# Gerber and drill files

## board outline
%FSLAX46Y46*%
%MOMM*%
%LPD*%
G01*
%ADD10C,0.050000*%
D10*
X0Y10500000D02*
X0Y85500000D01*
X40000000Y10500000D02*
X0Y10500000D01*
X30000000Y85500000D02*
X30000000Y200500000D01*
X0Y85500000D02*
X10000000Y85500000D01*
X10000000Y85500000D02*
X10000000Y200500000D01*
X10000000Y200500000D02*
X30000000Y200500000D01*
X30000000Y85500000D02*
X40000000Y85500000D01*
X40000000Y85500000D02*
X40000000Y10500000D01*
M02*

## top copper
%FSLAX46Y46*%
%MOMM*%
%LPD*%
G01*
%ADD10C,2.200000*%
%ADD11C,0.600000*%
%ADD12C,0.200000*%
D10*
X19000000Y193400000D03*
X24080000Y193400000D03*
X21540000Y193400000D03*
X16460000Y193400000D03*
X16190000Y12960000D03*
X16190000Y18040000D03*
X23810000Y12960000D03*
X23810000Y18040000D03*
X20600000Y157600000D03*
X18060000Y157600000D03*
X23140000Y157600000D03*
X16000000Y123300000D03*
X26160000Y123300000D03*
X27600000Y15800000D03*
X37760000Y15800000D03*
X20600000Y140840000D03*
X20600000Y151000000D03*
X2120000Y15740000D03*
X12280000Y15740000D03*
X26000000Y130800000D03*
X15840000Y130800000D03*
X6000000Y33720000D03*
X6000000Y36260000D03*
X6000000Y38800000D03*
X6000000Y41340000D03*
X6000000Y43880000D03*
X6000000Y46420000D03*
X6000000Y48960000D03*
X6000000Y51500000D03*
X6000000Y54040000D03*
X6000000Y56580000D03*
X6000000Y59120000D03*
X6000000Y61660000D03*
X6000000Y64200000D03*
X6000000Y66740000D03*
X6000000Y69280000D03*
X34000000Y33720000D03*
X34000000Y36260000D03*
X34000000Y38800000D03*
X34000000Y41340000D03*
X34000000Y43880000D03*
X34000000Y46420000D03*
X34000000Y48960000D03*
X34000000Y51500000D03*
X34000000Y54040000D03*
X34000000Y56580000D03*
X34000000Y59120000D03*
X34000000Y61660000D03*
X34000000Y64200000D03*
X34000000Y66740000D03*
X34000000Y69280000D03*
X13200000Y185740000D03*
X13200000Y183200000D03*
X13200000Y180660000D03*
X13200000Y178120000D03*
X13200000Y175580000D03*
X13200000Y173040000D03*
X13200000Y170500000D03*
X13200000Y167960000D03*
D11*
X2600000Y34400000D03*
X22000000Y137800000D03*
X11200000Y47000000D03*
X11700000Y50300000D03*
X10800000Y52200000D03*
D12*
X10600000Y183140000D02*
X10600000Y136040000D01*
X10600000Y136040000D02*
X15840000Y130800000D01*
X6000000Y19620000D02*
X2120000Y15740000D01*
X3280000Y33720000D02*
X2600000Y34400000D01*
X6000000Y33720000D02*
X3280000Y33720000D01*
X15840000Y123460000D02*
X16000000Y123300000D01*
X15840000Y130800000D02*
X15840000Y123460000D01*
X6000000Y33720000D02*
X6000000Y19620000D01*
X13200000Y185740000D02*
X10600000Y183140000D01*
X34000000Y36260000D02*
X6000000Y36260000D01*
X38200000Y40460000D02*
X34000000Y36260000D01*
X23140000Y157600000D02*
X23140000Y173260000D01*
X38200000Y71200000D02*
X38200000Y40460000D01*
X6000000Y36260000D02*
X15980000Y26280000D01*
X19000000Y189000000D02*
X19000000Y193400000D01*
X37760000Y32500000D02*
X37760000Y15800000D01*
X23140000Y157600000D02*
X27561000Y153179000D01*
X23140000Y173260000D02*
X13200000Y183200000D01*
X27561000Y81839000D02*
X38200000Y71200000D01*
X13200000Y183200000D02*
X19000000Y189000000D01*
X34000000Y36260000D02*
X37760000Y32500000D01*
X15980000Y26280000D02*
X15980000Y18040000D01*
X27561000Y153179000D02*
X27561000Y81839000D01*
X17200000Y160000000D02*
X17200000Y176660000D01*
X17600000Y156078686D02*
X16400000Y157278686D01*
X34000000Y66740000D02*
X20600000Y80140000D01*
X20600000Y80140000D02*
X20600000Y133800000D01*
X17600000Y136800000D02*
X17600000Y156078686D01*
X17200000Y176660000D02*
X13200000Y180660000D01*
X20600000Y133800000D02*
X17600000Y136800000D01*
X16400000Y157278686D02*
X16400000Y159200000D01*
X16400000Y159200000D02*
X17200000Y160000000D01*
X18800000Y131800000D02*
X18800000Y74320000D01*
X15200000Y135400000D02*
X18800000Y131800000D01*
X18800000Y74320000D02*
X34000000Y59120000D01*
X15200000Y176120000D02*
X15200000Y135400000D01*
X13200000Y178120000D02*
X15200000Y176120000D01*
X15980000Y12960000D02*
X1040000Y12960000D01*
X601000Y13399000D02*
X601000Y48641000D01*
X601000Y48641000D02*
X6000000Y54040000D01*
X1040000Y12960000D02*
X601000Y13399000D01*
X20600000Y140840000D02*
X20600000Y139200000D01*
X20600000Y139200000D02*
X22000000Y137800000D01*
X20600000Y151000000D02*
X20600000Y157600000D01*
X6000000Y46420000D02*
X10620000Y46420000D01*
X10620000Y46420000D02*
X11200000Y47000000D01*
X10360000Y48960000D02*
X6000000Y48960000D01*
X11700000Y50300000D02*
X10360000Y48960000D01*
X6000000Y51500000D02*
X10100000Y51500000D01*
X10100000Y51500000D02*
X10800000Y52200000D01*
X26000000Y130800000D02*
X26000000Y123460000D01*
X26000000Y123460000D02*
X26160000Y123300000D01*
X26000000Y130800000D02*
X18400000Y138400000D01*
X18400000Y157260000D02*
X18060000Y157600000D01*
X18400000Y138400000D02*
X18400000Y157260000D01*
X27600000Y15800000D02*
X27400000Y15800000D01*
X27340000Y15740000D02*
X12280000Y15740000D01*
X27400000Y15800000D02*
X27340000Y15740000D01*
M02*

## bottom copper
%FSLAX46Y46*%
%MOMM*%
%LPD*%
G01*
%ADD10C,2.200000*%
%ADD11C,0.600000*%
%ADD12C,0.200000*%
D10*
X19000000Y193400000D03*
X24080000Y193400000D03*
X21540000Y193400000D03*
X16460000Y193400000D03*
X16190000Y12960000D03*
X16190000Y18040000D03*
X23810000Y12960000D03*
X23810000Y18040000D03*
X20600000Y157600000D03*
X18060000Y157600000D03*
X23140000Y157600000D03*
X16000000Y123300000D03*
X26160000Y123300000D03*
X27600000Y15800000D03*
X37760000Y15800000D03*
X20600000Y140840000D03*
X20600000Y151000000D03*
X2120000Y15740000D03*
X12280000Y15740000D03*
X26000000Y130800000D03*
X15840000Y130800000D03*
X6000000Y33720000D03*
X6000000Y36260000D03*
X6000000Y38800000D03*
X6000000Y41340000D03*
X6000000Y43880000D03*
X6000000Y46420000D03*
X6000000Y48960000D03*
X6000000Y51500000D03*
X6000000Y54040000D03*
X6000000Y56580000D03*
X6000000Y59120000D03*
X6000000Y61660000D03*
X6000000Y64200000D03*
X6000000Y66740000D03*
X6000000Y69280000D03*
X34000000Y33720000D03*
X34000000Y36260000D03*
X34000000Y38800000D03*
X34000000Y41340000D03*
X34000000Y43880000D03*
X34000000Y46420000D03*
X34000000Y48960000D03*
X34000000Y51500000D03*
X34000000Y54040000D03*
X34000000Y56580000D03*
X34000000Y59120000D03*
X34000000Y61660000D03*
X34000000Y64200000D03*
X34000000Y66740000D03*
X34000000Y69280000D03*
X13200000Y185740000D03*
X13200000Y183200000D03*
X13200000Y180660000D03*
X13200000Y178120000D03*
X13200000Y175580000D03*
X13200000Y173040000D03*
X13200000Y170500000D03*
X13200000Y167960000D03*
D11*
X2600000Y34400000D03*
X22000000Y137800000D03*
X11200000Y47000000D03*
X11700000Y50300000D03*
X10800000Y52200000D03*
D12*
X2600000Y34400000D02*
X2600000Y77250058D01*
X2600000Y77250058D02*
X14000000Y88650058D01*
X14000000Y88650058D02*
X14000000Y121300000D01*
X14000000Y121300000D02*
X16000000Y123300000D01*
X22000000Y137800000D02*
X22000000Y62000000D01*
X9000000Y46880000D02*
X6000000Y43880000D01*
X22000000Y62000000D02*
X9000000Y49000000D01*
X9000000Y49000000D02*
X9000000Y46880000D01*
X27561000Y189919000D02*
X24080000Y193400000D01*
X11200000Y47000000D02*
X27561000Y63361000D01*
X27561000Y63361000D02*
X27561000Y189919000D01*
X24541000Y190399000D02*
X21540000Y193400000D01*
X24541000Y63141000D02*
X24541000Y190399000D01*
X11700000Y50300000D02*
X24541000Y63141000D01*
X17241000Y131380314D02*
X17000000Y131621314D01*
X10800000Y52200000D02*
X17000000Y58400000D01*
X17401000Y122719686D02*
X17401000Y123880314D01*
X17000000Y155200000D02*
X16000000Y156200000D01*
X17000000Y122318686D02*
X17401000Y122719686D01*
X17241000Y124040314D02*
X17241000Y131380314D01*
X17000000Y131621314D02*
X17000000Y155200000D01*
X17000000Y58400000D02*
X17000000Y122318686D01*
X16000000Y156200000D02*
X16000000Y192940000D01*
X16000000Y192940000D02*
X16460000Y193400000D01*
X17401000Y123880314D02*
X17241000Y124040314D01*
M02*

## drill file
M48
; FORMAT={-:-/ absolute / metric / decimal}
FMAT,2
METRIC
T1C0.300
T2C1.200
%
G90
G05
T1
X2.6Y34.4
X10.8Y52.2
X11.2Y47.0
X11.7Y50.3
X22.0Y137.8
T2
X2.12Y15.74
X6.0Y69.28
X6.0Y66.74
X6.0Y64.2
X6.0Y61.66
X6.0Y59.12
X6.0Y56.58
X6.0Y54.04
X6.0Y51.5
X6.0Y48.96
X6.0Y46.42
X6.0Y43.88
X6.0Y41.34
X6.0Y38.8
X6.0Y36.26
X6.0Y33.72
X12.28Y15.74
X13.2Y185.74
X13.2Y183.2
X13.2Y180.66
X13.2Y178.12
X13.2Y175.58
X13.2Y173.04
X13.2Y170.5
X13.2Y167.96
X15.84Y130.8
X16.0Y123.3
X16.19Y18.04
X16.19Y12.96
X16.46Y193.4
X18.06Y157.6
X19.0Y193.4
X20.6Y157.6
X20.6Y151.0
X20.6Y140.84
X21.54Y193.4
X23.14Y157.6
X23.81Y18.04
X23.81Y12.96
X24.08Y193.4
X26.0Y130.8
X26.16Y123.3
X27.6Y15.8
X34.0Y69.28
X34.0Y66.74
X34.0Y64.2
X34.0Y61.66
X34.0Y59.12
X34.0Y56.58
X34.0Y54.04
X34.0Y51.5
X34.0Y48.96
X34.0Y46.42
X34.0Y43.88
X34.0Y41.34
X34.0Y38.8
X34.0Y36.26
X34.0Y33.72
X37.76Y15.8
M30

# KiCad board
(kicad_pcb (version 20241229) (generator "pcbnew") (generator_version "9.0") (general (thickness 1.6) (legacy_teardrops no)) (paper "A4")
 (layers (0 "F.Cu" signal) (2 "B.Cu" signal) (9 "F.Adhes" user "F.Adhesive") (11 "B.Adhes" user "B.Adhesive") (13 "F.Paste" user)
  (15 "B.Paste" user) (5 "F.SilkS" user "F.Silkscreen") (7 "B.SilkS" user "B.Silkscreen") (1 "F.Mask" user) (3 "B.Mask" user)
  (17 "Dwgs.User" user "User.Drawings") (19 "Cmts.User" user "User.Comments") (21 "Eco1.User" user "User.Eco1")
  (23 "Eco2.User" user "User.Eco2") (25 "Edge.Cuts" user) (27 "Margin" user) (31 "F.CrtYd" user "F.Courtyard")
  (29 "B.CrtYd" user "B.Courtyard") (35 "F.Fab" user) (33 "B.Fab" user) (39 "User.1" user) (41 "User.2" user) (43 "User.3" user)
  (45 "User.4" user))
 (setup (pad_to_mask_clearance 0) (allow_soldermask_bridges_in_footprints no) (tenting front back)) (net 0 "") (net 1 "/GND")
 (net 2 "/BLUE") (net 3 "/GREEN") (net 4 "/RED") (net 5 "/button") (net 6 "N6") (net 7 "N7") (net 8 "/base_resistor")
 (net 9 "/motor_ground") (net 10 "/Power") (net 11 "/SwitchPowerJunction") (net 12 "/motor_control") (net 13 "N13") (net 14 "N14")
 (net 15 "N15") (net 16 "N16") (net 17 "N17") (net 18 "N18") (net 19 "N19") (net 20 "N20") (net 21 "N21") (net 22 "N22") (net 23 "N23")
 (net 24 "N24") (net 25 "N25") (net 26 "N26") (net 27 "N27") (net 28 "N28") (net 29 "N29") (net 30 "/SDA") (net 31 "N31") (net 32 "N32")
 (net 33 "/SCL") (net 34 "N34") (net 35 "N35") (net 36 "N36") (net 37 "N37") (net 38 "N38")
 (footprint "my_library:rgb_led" (layer "F.Cu") (at 16.46 -193.4)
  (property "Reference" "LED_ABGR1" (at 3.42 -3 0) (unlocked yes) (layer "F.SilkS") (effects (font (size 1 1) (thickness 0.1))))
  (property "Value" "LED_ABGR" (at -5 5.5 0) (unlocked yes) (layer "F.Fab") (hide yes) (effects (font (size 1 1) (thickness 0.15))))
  (pad "1" thru_hole circle (at 2.54 0) (size 2.2 2.2) (drill 1.2) (layers "*.Cu" "*.Mask") (remove_unused_layers no) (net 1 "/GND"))
  (pad "2" thru_hole circle (at 7.62 0) (size 2.2 2.2) (drill 1.2) (layers "*.Cu" "*.Mask") (remove_unused_layers no) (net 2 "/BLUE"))
  (pad "3" thru_hole circle (at 5.08 0) (size 2.2 2.2) (drill 1.2) (layers "*.Cu" "*.Mask") (remove_unused_layers no) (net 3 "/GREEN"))
  (pad "4" thru_hole circle (at 0 0) (size 2.2 2.2) (drill 1.2) (layers "*.Cu" "*.Mask") (remove_unused_layers no) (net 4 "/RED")))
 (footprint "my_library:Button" (layer "F.Cu") (at 16.19 -12.96 90)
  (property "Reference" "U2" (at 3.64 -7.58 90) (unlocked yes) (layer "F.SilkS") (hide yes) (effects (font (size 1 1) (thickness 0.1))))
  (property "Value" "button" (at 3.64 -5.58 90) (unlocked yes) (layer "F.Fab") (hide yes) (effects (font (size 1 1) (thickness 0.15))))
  (pad "1" thru_hole circle (at 0 0 90) (size 2.2 2.2) (drill 1.2) (layers "*.Cu" "*.Mask") (remove_unused_layers no) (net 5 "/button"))
  (pad "2" thru_hole circle (at 5.08 0 90) (size 2.2 2.2) (drill 1.2) (layers "*.Cu" "*.Mask") (remove_unused_layers no) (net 1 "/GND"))
  (pad "3" thru_hole circle (at 0 7.62 90) (size 2.2 2.2) (drill 1.2) (layers "*.Cu" "*.Mask") (remove_unused_layers no) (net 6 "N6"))
  (pad "4" thru_hole circle (at 5.08 7.62 90) (size 2.2 2.2) (drill 1.2) (layers "*.Cu" "*.Mask") (remove_unused_layers no) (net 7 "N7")))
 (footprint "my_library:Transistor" (layer "F.Cu") (at 18.06 -157.6 90)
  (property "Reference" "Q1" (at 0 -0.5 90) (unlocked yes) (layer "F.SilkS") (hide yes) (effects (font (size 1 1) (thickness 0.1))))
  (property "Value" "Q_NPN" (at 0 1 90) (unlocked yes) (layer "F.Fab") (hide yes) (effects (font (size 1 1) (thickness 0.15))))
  (pad "B" thru_hole circle (at 0 2.54 90) (size 2.2 2.2) (drill 1.2) (layers "*.Cu" "*.Mask") (remove_unused_layers no)
   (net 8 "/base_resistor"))
  (pad "C" thru_hole circle (at 0 0 90) (size 2.2 2.2) (drill 1.2) (layers "*.Cu" "*.Mask") (remove_unused_layers no)
   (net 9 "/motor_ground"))
  (pad "E" thru_hole circle (at 0 5.08 90) (size 2.2 2.2) (drill 1.2) (layers "*.Cu" "*.Mask") (remove_unused_layers no) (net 1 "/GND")))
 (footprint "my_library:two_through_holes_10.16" (layer "F.Cu") (at 16 -123.3)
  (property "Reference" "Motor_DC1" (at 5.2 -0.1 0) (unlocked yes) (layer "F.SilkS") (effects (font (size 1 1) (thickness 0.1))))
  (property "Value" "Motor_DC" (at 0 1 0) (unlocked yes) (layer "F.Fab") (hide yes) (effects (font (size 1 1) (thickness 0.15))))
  (pad "1" thru_hole circle (at 0 0) (size 2.2 2.2) (drill 1.2) (layers "*.Cu" "*.Mask") (remove_unused_layers no) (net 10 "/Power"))
  (pad "2" thru_hole circle (at 10.16 0) (size 2.2 2.2) (drill 1.2) (layers "*.Cu" "*.Mask") (remove_unused_layers no)
   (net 9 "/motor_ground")))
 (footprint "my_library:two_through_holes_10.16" (layer "F.Cu") (at 27.6 -15.8)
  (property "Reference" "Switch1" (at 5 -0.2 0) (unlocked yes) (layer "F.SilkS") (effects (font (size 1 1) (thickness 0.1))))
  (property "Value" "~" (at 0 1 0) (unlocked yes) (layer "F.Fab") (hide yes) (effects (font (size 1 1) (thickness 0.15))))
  (pad "1" thru_hole circle (at 0 0) (size 2.2 2.2) (drill 1.2) (layers "*.Cu" "*.Mask") (remove_unused_layers no)
   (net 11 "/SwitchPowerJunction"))
  (pad "2" thru_hole circle (at 10.16 0) (size 2.2 2.2) (drill 1.2) (layers "*.Cu" "*.Mask") (remove_unused_layers no) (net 1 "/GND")))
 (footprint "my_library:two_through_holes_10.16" (layer "F.Cu") (at 20.6 -140.84 90)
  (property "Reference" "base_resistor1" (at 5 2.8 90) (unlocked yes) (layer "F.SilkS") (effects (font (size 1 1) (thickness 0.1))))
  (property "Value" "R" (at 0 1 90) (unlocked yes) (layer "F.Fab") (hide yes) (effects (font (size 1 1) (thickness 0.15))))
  (pad "1" thru_hole circle (at 0 0 90) (size 2.2 2.2) (drill 1.2) (layers "*.Cu" "*.Mask") (remove_unused_layers no)
   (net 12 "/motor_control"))
  (pad "2" thru_hole circle (at 10.16 0 90) (size 2.2 2.2) (drill 1.2) (layers "*.Cu" "*.Mask") (remove_unused_layers no)
   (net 8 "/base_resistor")))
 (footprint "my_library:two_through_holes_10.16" (layer "F.Cu") (at 2.12 -15.74)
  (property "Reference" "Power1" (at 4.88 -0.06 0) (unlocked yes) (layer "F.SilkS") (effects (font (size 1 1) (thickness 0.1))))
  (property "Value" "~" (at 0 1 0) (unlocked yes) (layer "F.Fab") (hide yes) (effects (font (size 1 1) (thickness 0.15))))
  (pad "1" thru_hole circle (at 0 0) (size 2.2 2.2) (drill 1.2) (layers "*.Cu" "*.Mask") (remove_unused_layers no) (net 10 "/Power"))
  (pad "2" thru_hole circle (at 10.16 0) (size 2.2 2.2) (drill 1.2) (layers "*.Cu" "*.Mask") (remove_unused_layers no)
   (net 11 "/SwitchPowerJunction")))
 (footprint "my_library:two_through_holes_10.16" (layer "F.Cu") (at 26 -130.8 180)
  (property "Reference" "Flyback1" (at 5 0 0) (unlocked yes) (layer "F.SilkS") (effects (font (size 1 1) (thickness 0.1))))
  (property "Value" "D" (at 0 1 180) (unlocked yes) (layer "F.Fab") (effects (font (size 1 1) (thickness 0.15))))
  (pad "1" thru_hole circle (at 0 0 180) (size 2.2 2.2) (drill 1.2) (layers "*.Cu" "*.Mask") (remove_unused_layers no)
   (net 9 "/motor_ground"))
  (pad "2" thru_hole circle (at 10.16 0 180) (size 2.2 2.2) (drill 1.2) (layers "*.Cu" "*.Mask") (remove_unused_layers no) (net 10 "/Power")))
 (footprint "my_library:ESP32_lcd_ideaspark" (layer "F.Cu") (at 20 -51.5)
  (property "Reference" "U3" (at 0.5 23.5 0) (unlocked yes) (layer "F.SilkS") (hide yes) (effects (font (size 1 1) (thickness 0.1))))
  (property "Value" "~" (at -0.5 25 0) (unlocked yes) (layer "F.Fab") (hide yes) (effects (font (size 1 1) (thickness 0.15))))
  (pad "1" thru_hole circle (at -14 17.78) (size 2.2 2.2) (drill 1.2) (layers "*.Cu" "*.Mask") (remove_unused_layers no) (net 10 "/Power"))
  (pad "2" thru_hole circle (at -14 15.24) (size 2.2 2.2) (drill 1.2) (layers "*.Cu" "*.Mask") (remove_unused_layers no) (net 1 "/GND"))
  (pad "3" thru_hole circle (at -14 12.7) (size 2.2 2.2) (drill 1.2) (layers "*.Cu" "*.Mask") (remove_unused_layers no) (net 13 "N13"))
  (pad "4" thru_hole circle (at -14 10.16) (size 2.2 2.2) (drill 1.2) (layers "*.Cu" "*.Mask") (remove_unused_layers no) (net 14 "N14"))
  (pad "5" thru_hole circle (at -14 7.62) (size 2.2 2.2) (drill 1.2) (layers "*.Cu" "*.Mask") (remove_unused_layers no)
   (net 12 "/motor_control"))
  (pad "6" thru_hole circle (at -14 5.08) (size 2.2 2.2) (drill 1.2) (layers "*.Cu" "*.Mask") (remove_unused_layers no) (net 2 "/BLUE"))
  (pad "7" thru_hole circle (at -14 2.54) (size 2.2 2.2) (drill 1.2) (layers "*.Cu" "*.Mask") (remove_unused_layers no) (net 3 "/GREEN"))
  (pad "8" thru_hole circle (at -14 0) (size 2.2 2.2) (drill 1.2) (layers "*.Cu" "*.Mask") (remove_unused_layers no) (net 4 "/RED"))
  (pad "9" thru_hole circle (at -14 -2.54) (size 2.2 2.2) (drill 1.2) (layers "*.Cu" "*.Mask") (remove_unused_layers no) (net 5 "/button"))
  (pad "10" thru_hole circle (at -14 -5.08) (size 2.2 2.2) (drill 1.2) (layers "*.Cu" "*.Mask") (remove_unused_layers no) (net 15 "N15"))
  (pad "11" thru_hole circle (at -14 -7.62) (size 2.2 2.2) (drill 1.2) (layers "*.Cu" "*.Mask") (remove_unused_layers no) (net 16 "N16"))
  (pad "12" thru_hole circle (at -14 -10.16) (size 2.2 2.2) (drill 1.2) (layers "*.Cu" "*.Mask") (remove_unused_layers no) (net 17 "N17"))
  (pad "13" thru_hole circle (at -14 -12.7) (size 2.2 2.2) (drill 1.2) (layers "*.Cu" "*.Mask") (remove_unused_layers no) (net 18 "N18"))
  (pad "14" thru_hole circle (at -14 -15.24) (size 2.2 2.2) (drill 1.2) (layers "*.Cu" "*.Mask") (remove_unused_layers no) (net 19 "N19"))
  (pad "15" thru_hole circle (at -14 -17.78) (size 2.2 2.2) (drill 1.2) (layers "*.Cu" "*.Mask") (remove_unused_layers no) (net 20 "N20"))
  (pad "16" thru_hole circle (at 14 17.78) (size 2.2 2.2) (drill 1.2) (layers "*.Cu" "*.Mask") (remove_unused_layers no) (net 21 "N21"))
  (pad "17" thru_hole circle (at 14 15.24) (size 2.2 2.2) (drill 1.2) (layers "*.Cu" "*.Mask") (remove_unused_layers no) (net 1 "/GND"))
  (pad "18" thru_hole circle (at 14 12.7) (size 2.2 2.2) (drill 1.2) (layers "*.Cu" "*.Mask") (remove_unused_layers no) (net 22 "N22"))
  (pad "19" thru_hole circle (at 14 10.16) (size 2.2 2.2) (drill 1.2) (layers "*.Cu" "*.Mask") (remove_unused_layers no) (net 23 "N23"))
  (pad "20" thru_hole circle (at 14 7.62) (size 2.2 2.2) (drill 1.2) (layers "*.Cu" "*.Mask") (remove_unused_layers no) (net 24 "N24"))
  (pad "21" thru_hole circle (at 14 5.08) (size 2.2 2.2) (drill 1.2) (layers "*.Cu" "*.Mask") (remove_unused_layers no) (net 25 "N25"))
  (pad "22" thru_hole circle (at 14 2.54) (size 2.2 2.2) (drill 1.2) (layers "*.Cu" "*.Mask") (remove_unused_layers no) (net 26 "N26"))
  (pad "23" thru_hole circle (at 14 0) (size 2.2 2.2) (drill 1.2) (layers "*.Cu" "*.Mask") (remove_unused_layers no) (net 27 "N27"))
  (pad "24" thru_hole circle (at 14 -2.54) (size 2.2 2.2) (drill 1.2) (layers "*.Cu" "*.Mask") (remove_unused_layers no) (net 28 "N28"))
  (pad "25" thru_hole circle (at 14 -5.08) (size 2.2 2.2) (drill 1.2) (layers "*.Cu" "*.Mask") (remove_unused_layers no) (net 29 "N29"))
  (pad "26" thru_hole circle (at 14 -7.62) (size 2.2 2.2) (drill 1.2) (layers "*.Cu" "*.Mask") (remove_unused_layers no) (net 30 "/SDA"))
  (pad "27" thru_hole circle (at 14 -10.16) (size 2.2 2.2) (drill 1.2) (layers "*.Cu" "*.Mask") (remove_unused_layers no) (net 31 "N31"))
  (pad "28" thru_hole circle (at 14 -12.7) (size 2.2 2.2) (drill 1.2) (layers "*.Cu" "*.Mask") (remove_unused_layers no) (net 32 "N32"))
  (pad "29" thru_hole circle (at 14 -15.24) (size 2.2 2.2) (drill 1.2) (layers "*.Cu" "*.Mask") (remove_unused_layers no) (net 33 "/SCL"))
  (pad "30" thru_hole circle (at 14 -17.78) (size 2.2 2.2) (drill 1.2) (layers "*.Cu" "*.Mask") (remove_unused_layers no) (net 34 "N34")))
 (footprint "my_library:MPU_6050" (layer "F.Cu") (at 13.2 -185.74)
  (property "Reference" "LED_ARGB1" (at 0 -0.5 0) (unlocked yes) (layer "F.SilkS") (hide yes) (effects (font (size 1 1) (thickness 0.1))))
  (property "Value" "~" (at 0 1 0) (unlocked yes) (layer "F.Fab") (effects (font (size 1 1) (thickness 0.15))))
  (pad "1" thru_hole circle (at 0 0) (size 2.2 2.2) (drill 1.2) (layers "*.Cu" "*.Mask") (remove_unused_layers no) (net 10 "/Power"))
  (pad "2" thru_hole circle (at 0 2.54) (size 2.2 2.2) (drill 1.2) (layers "*.Cu" "*.Mask") (remove_unused_layers no) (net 1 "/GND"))
  (pad "3" thru_hole circle (at 0 5.08) (size 2.2 2.2) (drill 1.2) (layers "*.Cu" "*.Mask") (remove_unused_layers no) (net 33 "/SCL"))
  (pad "4" thru_hole circle (at 0 7.62) (size 2.2 2.2) (drill 1.2) (layers "*.Cu" "*.Mask") (remove_unused_layers no) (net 30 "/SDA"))
  (pad "5" thru_hole circle (at 0 10.16) (size 2.2 2.2) (drill 1.2) (layers "*.Cu" "*.Mask") (remove_unused_layers no) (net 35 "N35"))
  (pad "6" thru_hole circle (at 0 12.7) (size 2.2 2.2) (drill 1.2) (layers "*.Cu" "*.Mask") (remove_unused_layers no) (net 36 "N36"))
  (pad "7" thru_hole circle (at 0 15.24) (size 2.2 2.2) (drill 1.2) (layers "*.Cu" "*.Mask") (remove_unused_layers no) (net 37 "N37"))
  (pad "8" thru_hole circle (at 0 17.78) (size 2.2 2.2) (drill 1.2) (layers "*.Cu" "*.Mask") (remove_unused_layers no) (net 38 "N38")))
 (gr_line (start 0 -10.5) (end 0 -85.5) (stroke (width 0.05) (type solid)) (layer "Edge.Cuts"))
 (gr_line (start 40 -10.5) (end 0 -10.5) (stroke (width 0.05) (type solid)) (layer "Edge.Cuts"))
 (gr_line (start 30 -85.5) (end 30 -200.5) (stroke (width 0.05) (type solid)) (layer "Edge.Cuts"))
 (gr_line (start 0 -85.5) (end 10 -85.5) (stroke (width 0.05) (type default)) (layer "Edge.Cuts"))
 (gr_line (start 10 -85.5) (end 10 -200.5) (stroke (width 0.05) (type solid)) (layer "Edge.Cuts"))
 (gr_line (start 10 -200.5) (end 30 -200.5) (stroke (width 0.05) (type solid)) (layer "Edge.Cuts"))
 (gr_line (start 30 -85.5) (end 40 -85.5) (stroke (width 0.05) (type default)) (layer "Edge.Cuts"))
 (gr_line (start 40 -85.5) (end 40 -10.5) (stroke (width 0.05) (type solid)) (layer "Edge.Cuts"))
 (segment (start 10.6 -183.14) (end 10.6 -136.04) (width 0.2) (layer "F.Cu") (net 10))
 (segment (start 10.6 -136.04) (end 15.84 -130.8) (width 0.2) (layer "F.Cu") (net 10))
 (segment (start 6 -19.62) (end 2.12 -15.74) (width 0.2) (layer "F.Cu") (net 10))
 (segment (start 3.28 -33.72) (end 2.6 -34.4) (width 0.2) (layer "F.Cu") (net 10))
 (segment (start 6 -33.72) (end 3.28 -33.72) (width 0.2) (layer "F.Cu") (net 10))
 (segment (start 15.84 -123.46) (end 16 -123.3) (width 0.2) (layer "F.Cu") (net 10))
 (segment (start 15.84 -130.8) (end 15.84 -123.46) (width 0.2) (layer "F.Cu") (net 10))
 (segment (start 6 -33.72) (end 6 -19.62) (width 0.2) (layer "F.Cu") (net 10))
 (segment (start 13.2 -185.74) (end 10.6 -183.14) (width 0.2) (layer "F.Cu") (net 10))
 (via (at 2.6 -34.4) (size 0.6) (drill 0.3) (layers "F.Cu" "B.Cu") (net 10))
 (segment (start 2.6 -34.4) (end 2.6 -77.250058) (width 0.2) (layer "B.Cu") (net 10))
 (segment (start 2.6 -77.250058) (end 14 -88.650058) (width 0.2) (layer "B.Cu") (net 10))
 (segment (start 14 -88.650058) (end 14 -121.3) (width 0.2) (layer "B.Cu") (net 10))
 (segment (start 14 -121.3) (end 16 -123.3) (width 0.2) (layer "B.Cu") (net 10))
 (segment (start 34 -36.26) (end 6 -36.26) (width 0.2) (layer "F.Cu") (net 1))
 (segment (start 38.2 -40.46) (end 34 -36.26) (width 0.2) (layer "F.Cu") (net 1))
 (segment (start 23.14 -157.6) (end 23.14 -173.26) (width 0.2) (layer "F.Cu") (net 1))
 (segment (start 38.2 -71.2) (end 38.2 -40.46) (width 0.2) (layer "F.Cu") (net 1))
 (segment (start 6 -36.26) (end 15.98 -26.28) (width 0.2) (layer "F.Cu") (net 1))
 (segment (start 19 -189) (end 19 -193.4) (width 0.2) (layer "F.Cu") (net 1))
 (segment (start 37.76 -32.5) (end 37.76 -15.8) (width 0.2) (layer "F.Cu") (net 1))
 (segment (start 23.14 -157.6) (end 27.561 -153.179) (width 0.2) (layer "F.Cu") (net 1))
 (segment (start 23.14 -173.26) (end 13.2 -183.2) (width 0.2) (layer "F.Cu") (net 1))
 (segment (start 27.561 -81.839) (end 38.2 -71.2) (width 0.2) (layer "F.Cu") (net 1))
 (segment (start 13.2 -183.2) (end 19 -189) (width 0.2) (layer "F.Cu") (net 1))
 (segment (start 34 -36.26) (end 37.76 -32.5) (width 0.2) (layer "F.Cu") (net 1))
 (segment (start 15.98 -26.28) (end 15.98 -18.04) (width 0.2) (layer "F.Cu") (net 1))
 (segment (start 27.561 -153.179) (end 27.561 -81.839) (width 0.2) (layer "F.Cu") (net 1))
 (segment (start 17.2 -160) (end 17.2 -176.66) (width 0.2) (layer "F.Cu") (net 33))
 (segment (start 17.6 -156.078686) (end 16.4 -157.278686) (width 0.2) (layer "F.Cu") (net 33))
 (segment (start 34 -66.74) (end 20.6 -80.14) (width 0.2) (layer "F.Cu") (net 33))
 (segment (start 20.6 -80.14) (end 20.6 -133.8) (width 0.2) (layer "F.Cu") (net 33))
 (segment (start 17.6 -136.8) (end 17.6 -156.078686) (width 0.2) (layer "F.Cu") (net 33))
 (segment (start 17.2 -176.66) (end 13.2 -180.66) (width 0.2) (layer "F.Cu") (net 33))
 (segment (start 20.6 -133.8) (end 17.6 -136.8) (width 0.2) (layer "F.Cu") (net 33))
 (segment (start 16.4 -157.278686) (end 16.4 -159.2) (width 0.2) (layer "F.Cu") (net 33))
 (segment (start 16.4 -159.2) (end 17.2 -160) (width 0.2) (layer "F.Cu") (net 33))
 (segment (start 18.8 -131.8) (end 18.8 -74.32) (width 0.2) (layer "F.Cu") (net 30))
 (segment (start 15.2 -135.4) (end 18.8 -131.8) (width 0.2) (layer "F.Cu") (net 30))
 (segment (start 18.8 -74.32) (end 34 -59.12) (width 0.2) (layer "F.Cu") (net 30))
 (segment (start 15.2 -176.12) (end 15.2 -135.4) (width 0.2) (layer "F.Cu") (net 30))
 (segment (start 13.2 -178.12) (end 15.2 -176.12) (width 0.2) (layer "F.Cu") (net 30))
 (segment (start 15.98 -12.96) (end 1.04 -12.96) (width 0.2) (layer "F.Cu") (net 5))
 (segment (start 0.601 -13.399) (end 0.601 -48.641) (width 0.2) (layer "F.Cu") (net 5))
 (segment (start 0.601 -48.641) (end 6 -54.04) (width 0.2) (layer "F.Cu") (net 5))
 (segment (start 1.04 -12.96) (end 0.601 -13.399) (width 0.2) (layer "F.Cu") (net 5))
 (segment (start 20.6 -140.84) (end 20.6 -139.2) (width 0.2) (layer "F.Cu") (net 12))
 (segment (start 20.6 -139.2) (end 22 -137.8) (width 0.2) (layer "F.Cu") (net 12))
 (via (at 22 -137.8) (size 0.6) (drill 0.3) (layers "F.Cu" "B.Cu") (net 12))
 (segment (start 22 -137.8) (end 22 -62) (width 0.2) (layer "B.Cu") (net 12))
 (segment (start 9 -46.88) (end 6 -43.88) (width 0.2) (layer "B.Cu") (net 12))
 (segment (start 22 -62) (end 9 -49) (width 0.2) (layer "B.Cu") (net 12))
 (segment (start 9 -49) (end 9 -46.88) (width 0.2) (layer "B.Cu") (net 12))
 (segment (start 20.6 -151) (end 20.6 -157.6) (width 0.2) (layer "F.Cu") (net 8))
 (segment (start 6 -46.42) (end 10.62 -46.42) (width 0.2) (layer "F.Cu") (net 2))
 (segment (start 10.62 -46.42) (end 11.2 -47) (width 0.2) (layer "F.Cu") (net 2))
 (via (at 11.2 -47) (size 0.6) (drill 0.3) (layers "F.Cu" "B.Cu") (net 2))
 (segment (start 27.561 -189.919) (end 24.08 -193.4) (width 0.2) (layer "B.Cu") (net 2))
 (segment (start 11.2 -47) (end 27.561 -63.361) (width 0.2) (layer "B.Cu") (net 2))
 (segment (start 27.561 -63.361) (end 27.561 -189.919) (width 0.2) (layer "B.Cu") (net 2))
 (segment (start 10.36 -48.96) (end 6 -48.96) (width 0.2) (layer "F.Cu") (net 3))
 (segment (start 11.7 -50.3) (end 10.36 -48.96) (width 0.2) (layer "F.Cu") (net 3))
 (via (at 11.7 -50.3) (size 0.6) (drill 0.3) (layers "F.Cu" "B.Cu") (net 3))
 (segment (start 24.541 -190.399) (end 21.54 -193.4) (width 0.2) (layer "B.Cu") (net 3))
 (segment (start 24.541 -63.141) (end 24.541 -190.399) (width 0.2) (layer "B.Cu") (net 3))
 (segment (start 11.7 -50.3) (end 24.541 -63.141) (width 0.2) (layer "B.Cu") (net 3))
 (segment (start 6 -51.5) (end 10.1 -51.5) (width 0.2) (layer "F.Cu") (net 4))
 (segment (start 10.1 -51.5) (end 10.8 -52.2) (width 0.2) (layer "F.Cu") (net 4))
 (via (at 10.8 -52.2) (size 0.6) (drill 0.3) (layers "F.Cu" "B.Cu") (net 4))
 (segment (start 17.241 -131.380314) (end 17 -131.621314) (width 0.2) (layer "B.Cu") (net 4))
 (segment (start 10.8 -52.2) (end 17 -58.4) (width 0.2) (layer "B.Cu") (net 4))
 (segment (start 17.401 -122.719686) (end 17.401 -123.880314) (width 0.2) (layer "B.Cu") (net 4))
 (segment (start 17 -155.2) (end 16 -156.2) (width 0.2) (layer "B.Cu") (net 4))
 (segment (start 17 -122.318686) (end 17.401 -122.719686) (width 0.2) (layer "B.Cu") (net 4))
 (segment (start 17.241 -124.040314) (end 17.241 -131.380314) (width 0.2) (layer "B.Cu") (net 4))
 (segment (start 17 -131.621314) (end 17 -155.2) (width 0.2) (layer "B.Cu") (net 4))
 (segment (start 17 -58.4) (end 17 -122.318686) (width 0.2) (layer "B.Cu") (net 4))
 (segment (start 16 -156.2) (end 16 -192.94) (width 0.2) (layer "B.Cu") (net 4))
 (segment (start 16 -192.94) (end 16.46 -193.4) (width 0.2) (layer "B.Cu") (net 4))
 (segment (start 17.401 -123.880314) (end 17.241 -124.040314) (width 0.2) (layer "B.Cu") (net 4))
 (segment (start 26 -130.8) (end 26 -123.46) (width 0.2) (layer "F.Cu") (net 9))
 (segment (start 26 -123.46) (end 26.16 -123.3) (width 0.2) (layer "F.Cu") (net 9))
 (segment (start 26 -130.8) (end 18.4 -138.4) (width 0.2) (layer "F.Cu") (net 9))
 (segment (start 18.4 -157.26) (end 18.06 -157.6) (width 0.2) (layer "F.Cu") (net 9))
 (segment (start 18.4 -138.4) (end 18.4 -157.26) (width 0.2) (layer "F.Cu") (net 9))
 (segment (start 27.6 -15.8) (end 27.4 -15.8) (width 0.2) (layer "F.Cu") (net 11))
 (segment (start 27.34 -15.74) (end 12.28 -15.74) (width 0.2) (layer "F.Cu") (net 11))
 (segment (start 27.4 -15.8) (end 27.34 -15.74) (width 0.2) (layer "F.Cu") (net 11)))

